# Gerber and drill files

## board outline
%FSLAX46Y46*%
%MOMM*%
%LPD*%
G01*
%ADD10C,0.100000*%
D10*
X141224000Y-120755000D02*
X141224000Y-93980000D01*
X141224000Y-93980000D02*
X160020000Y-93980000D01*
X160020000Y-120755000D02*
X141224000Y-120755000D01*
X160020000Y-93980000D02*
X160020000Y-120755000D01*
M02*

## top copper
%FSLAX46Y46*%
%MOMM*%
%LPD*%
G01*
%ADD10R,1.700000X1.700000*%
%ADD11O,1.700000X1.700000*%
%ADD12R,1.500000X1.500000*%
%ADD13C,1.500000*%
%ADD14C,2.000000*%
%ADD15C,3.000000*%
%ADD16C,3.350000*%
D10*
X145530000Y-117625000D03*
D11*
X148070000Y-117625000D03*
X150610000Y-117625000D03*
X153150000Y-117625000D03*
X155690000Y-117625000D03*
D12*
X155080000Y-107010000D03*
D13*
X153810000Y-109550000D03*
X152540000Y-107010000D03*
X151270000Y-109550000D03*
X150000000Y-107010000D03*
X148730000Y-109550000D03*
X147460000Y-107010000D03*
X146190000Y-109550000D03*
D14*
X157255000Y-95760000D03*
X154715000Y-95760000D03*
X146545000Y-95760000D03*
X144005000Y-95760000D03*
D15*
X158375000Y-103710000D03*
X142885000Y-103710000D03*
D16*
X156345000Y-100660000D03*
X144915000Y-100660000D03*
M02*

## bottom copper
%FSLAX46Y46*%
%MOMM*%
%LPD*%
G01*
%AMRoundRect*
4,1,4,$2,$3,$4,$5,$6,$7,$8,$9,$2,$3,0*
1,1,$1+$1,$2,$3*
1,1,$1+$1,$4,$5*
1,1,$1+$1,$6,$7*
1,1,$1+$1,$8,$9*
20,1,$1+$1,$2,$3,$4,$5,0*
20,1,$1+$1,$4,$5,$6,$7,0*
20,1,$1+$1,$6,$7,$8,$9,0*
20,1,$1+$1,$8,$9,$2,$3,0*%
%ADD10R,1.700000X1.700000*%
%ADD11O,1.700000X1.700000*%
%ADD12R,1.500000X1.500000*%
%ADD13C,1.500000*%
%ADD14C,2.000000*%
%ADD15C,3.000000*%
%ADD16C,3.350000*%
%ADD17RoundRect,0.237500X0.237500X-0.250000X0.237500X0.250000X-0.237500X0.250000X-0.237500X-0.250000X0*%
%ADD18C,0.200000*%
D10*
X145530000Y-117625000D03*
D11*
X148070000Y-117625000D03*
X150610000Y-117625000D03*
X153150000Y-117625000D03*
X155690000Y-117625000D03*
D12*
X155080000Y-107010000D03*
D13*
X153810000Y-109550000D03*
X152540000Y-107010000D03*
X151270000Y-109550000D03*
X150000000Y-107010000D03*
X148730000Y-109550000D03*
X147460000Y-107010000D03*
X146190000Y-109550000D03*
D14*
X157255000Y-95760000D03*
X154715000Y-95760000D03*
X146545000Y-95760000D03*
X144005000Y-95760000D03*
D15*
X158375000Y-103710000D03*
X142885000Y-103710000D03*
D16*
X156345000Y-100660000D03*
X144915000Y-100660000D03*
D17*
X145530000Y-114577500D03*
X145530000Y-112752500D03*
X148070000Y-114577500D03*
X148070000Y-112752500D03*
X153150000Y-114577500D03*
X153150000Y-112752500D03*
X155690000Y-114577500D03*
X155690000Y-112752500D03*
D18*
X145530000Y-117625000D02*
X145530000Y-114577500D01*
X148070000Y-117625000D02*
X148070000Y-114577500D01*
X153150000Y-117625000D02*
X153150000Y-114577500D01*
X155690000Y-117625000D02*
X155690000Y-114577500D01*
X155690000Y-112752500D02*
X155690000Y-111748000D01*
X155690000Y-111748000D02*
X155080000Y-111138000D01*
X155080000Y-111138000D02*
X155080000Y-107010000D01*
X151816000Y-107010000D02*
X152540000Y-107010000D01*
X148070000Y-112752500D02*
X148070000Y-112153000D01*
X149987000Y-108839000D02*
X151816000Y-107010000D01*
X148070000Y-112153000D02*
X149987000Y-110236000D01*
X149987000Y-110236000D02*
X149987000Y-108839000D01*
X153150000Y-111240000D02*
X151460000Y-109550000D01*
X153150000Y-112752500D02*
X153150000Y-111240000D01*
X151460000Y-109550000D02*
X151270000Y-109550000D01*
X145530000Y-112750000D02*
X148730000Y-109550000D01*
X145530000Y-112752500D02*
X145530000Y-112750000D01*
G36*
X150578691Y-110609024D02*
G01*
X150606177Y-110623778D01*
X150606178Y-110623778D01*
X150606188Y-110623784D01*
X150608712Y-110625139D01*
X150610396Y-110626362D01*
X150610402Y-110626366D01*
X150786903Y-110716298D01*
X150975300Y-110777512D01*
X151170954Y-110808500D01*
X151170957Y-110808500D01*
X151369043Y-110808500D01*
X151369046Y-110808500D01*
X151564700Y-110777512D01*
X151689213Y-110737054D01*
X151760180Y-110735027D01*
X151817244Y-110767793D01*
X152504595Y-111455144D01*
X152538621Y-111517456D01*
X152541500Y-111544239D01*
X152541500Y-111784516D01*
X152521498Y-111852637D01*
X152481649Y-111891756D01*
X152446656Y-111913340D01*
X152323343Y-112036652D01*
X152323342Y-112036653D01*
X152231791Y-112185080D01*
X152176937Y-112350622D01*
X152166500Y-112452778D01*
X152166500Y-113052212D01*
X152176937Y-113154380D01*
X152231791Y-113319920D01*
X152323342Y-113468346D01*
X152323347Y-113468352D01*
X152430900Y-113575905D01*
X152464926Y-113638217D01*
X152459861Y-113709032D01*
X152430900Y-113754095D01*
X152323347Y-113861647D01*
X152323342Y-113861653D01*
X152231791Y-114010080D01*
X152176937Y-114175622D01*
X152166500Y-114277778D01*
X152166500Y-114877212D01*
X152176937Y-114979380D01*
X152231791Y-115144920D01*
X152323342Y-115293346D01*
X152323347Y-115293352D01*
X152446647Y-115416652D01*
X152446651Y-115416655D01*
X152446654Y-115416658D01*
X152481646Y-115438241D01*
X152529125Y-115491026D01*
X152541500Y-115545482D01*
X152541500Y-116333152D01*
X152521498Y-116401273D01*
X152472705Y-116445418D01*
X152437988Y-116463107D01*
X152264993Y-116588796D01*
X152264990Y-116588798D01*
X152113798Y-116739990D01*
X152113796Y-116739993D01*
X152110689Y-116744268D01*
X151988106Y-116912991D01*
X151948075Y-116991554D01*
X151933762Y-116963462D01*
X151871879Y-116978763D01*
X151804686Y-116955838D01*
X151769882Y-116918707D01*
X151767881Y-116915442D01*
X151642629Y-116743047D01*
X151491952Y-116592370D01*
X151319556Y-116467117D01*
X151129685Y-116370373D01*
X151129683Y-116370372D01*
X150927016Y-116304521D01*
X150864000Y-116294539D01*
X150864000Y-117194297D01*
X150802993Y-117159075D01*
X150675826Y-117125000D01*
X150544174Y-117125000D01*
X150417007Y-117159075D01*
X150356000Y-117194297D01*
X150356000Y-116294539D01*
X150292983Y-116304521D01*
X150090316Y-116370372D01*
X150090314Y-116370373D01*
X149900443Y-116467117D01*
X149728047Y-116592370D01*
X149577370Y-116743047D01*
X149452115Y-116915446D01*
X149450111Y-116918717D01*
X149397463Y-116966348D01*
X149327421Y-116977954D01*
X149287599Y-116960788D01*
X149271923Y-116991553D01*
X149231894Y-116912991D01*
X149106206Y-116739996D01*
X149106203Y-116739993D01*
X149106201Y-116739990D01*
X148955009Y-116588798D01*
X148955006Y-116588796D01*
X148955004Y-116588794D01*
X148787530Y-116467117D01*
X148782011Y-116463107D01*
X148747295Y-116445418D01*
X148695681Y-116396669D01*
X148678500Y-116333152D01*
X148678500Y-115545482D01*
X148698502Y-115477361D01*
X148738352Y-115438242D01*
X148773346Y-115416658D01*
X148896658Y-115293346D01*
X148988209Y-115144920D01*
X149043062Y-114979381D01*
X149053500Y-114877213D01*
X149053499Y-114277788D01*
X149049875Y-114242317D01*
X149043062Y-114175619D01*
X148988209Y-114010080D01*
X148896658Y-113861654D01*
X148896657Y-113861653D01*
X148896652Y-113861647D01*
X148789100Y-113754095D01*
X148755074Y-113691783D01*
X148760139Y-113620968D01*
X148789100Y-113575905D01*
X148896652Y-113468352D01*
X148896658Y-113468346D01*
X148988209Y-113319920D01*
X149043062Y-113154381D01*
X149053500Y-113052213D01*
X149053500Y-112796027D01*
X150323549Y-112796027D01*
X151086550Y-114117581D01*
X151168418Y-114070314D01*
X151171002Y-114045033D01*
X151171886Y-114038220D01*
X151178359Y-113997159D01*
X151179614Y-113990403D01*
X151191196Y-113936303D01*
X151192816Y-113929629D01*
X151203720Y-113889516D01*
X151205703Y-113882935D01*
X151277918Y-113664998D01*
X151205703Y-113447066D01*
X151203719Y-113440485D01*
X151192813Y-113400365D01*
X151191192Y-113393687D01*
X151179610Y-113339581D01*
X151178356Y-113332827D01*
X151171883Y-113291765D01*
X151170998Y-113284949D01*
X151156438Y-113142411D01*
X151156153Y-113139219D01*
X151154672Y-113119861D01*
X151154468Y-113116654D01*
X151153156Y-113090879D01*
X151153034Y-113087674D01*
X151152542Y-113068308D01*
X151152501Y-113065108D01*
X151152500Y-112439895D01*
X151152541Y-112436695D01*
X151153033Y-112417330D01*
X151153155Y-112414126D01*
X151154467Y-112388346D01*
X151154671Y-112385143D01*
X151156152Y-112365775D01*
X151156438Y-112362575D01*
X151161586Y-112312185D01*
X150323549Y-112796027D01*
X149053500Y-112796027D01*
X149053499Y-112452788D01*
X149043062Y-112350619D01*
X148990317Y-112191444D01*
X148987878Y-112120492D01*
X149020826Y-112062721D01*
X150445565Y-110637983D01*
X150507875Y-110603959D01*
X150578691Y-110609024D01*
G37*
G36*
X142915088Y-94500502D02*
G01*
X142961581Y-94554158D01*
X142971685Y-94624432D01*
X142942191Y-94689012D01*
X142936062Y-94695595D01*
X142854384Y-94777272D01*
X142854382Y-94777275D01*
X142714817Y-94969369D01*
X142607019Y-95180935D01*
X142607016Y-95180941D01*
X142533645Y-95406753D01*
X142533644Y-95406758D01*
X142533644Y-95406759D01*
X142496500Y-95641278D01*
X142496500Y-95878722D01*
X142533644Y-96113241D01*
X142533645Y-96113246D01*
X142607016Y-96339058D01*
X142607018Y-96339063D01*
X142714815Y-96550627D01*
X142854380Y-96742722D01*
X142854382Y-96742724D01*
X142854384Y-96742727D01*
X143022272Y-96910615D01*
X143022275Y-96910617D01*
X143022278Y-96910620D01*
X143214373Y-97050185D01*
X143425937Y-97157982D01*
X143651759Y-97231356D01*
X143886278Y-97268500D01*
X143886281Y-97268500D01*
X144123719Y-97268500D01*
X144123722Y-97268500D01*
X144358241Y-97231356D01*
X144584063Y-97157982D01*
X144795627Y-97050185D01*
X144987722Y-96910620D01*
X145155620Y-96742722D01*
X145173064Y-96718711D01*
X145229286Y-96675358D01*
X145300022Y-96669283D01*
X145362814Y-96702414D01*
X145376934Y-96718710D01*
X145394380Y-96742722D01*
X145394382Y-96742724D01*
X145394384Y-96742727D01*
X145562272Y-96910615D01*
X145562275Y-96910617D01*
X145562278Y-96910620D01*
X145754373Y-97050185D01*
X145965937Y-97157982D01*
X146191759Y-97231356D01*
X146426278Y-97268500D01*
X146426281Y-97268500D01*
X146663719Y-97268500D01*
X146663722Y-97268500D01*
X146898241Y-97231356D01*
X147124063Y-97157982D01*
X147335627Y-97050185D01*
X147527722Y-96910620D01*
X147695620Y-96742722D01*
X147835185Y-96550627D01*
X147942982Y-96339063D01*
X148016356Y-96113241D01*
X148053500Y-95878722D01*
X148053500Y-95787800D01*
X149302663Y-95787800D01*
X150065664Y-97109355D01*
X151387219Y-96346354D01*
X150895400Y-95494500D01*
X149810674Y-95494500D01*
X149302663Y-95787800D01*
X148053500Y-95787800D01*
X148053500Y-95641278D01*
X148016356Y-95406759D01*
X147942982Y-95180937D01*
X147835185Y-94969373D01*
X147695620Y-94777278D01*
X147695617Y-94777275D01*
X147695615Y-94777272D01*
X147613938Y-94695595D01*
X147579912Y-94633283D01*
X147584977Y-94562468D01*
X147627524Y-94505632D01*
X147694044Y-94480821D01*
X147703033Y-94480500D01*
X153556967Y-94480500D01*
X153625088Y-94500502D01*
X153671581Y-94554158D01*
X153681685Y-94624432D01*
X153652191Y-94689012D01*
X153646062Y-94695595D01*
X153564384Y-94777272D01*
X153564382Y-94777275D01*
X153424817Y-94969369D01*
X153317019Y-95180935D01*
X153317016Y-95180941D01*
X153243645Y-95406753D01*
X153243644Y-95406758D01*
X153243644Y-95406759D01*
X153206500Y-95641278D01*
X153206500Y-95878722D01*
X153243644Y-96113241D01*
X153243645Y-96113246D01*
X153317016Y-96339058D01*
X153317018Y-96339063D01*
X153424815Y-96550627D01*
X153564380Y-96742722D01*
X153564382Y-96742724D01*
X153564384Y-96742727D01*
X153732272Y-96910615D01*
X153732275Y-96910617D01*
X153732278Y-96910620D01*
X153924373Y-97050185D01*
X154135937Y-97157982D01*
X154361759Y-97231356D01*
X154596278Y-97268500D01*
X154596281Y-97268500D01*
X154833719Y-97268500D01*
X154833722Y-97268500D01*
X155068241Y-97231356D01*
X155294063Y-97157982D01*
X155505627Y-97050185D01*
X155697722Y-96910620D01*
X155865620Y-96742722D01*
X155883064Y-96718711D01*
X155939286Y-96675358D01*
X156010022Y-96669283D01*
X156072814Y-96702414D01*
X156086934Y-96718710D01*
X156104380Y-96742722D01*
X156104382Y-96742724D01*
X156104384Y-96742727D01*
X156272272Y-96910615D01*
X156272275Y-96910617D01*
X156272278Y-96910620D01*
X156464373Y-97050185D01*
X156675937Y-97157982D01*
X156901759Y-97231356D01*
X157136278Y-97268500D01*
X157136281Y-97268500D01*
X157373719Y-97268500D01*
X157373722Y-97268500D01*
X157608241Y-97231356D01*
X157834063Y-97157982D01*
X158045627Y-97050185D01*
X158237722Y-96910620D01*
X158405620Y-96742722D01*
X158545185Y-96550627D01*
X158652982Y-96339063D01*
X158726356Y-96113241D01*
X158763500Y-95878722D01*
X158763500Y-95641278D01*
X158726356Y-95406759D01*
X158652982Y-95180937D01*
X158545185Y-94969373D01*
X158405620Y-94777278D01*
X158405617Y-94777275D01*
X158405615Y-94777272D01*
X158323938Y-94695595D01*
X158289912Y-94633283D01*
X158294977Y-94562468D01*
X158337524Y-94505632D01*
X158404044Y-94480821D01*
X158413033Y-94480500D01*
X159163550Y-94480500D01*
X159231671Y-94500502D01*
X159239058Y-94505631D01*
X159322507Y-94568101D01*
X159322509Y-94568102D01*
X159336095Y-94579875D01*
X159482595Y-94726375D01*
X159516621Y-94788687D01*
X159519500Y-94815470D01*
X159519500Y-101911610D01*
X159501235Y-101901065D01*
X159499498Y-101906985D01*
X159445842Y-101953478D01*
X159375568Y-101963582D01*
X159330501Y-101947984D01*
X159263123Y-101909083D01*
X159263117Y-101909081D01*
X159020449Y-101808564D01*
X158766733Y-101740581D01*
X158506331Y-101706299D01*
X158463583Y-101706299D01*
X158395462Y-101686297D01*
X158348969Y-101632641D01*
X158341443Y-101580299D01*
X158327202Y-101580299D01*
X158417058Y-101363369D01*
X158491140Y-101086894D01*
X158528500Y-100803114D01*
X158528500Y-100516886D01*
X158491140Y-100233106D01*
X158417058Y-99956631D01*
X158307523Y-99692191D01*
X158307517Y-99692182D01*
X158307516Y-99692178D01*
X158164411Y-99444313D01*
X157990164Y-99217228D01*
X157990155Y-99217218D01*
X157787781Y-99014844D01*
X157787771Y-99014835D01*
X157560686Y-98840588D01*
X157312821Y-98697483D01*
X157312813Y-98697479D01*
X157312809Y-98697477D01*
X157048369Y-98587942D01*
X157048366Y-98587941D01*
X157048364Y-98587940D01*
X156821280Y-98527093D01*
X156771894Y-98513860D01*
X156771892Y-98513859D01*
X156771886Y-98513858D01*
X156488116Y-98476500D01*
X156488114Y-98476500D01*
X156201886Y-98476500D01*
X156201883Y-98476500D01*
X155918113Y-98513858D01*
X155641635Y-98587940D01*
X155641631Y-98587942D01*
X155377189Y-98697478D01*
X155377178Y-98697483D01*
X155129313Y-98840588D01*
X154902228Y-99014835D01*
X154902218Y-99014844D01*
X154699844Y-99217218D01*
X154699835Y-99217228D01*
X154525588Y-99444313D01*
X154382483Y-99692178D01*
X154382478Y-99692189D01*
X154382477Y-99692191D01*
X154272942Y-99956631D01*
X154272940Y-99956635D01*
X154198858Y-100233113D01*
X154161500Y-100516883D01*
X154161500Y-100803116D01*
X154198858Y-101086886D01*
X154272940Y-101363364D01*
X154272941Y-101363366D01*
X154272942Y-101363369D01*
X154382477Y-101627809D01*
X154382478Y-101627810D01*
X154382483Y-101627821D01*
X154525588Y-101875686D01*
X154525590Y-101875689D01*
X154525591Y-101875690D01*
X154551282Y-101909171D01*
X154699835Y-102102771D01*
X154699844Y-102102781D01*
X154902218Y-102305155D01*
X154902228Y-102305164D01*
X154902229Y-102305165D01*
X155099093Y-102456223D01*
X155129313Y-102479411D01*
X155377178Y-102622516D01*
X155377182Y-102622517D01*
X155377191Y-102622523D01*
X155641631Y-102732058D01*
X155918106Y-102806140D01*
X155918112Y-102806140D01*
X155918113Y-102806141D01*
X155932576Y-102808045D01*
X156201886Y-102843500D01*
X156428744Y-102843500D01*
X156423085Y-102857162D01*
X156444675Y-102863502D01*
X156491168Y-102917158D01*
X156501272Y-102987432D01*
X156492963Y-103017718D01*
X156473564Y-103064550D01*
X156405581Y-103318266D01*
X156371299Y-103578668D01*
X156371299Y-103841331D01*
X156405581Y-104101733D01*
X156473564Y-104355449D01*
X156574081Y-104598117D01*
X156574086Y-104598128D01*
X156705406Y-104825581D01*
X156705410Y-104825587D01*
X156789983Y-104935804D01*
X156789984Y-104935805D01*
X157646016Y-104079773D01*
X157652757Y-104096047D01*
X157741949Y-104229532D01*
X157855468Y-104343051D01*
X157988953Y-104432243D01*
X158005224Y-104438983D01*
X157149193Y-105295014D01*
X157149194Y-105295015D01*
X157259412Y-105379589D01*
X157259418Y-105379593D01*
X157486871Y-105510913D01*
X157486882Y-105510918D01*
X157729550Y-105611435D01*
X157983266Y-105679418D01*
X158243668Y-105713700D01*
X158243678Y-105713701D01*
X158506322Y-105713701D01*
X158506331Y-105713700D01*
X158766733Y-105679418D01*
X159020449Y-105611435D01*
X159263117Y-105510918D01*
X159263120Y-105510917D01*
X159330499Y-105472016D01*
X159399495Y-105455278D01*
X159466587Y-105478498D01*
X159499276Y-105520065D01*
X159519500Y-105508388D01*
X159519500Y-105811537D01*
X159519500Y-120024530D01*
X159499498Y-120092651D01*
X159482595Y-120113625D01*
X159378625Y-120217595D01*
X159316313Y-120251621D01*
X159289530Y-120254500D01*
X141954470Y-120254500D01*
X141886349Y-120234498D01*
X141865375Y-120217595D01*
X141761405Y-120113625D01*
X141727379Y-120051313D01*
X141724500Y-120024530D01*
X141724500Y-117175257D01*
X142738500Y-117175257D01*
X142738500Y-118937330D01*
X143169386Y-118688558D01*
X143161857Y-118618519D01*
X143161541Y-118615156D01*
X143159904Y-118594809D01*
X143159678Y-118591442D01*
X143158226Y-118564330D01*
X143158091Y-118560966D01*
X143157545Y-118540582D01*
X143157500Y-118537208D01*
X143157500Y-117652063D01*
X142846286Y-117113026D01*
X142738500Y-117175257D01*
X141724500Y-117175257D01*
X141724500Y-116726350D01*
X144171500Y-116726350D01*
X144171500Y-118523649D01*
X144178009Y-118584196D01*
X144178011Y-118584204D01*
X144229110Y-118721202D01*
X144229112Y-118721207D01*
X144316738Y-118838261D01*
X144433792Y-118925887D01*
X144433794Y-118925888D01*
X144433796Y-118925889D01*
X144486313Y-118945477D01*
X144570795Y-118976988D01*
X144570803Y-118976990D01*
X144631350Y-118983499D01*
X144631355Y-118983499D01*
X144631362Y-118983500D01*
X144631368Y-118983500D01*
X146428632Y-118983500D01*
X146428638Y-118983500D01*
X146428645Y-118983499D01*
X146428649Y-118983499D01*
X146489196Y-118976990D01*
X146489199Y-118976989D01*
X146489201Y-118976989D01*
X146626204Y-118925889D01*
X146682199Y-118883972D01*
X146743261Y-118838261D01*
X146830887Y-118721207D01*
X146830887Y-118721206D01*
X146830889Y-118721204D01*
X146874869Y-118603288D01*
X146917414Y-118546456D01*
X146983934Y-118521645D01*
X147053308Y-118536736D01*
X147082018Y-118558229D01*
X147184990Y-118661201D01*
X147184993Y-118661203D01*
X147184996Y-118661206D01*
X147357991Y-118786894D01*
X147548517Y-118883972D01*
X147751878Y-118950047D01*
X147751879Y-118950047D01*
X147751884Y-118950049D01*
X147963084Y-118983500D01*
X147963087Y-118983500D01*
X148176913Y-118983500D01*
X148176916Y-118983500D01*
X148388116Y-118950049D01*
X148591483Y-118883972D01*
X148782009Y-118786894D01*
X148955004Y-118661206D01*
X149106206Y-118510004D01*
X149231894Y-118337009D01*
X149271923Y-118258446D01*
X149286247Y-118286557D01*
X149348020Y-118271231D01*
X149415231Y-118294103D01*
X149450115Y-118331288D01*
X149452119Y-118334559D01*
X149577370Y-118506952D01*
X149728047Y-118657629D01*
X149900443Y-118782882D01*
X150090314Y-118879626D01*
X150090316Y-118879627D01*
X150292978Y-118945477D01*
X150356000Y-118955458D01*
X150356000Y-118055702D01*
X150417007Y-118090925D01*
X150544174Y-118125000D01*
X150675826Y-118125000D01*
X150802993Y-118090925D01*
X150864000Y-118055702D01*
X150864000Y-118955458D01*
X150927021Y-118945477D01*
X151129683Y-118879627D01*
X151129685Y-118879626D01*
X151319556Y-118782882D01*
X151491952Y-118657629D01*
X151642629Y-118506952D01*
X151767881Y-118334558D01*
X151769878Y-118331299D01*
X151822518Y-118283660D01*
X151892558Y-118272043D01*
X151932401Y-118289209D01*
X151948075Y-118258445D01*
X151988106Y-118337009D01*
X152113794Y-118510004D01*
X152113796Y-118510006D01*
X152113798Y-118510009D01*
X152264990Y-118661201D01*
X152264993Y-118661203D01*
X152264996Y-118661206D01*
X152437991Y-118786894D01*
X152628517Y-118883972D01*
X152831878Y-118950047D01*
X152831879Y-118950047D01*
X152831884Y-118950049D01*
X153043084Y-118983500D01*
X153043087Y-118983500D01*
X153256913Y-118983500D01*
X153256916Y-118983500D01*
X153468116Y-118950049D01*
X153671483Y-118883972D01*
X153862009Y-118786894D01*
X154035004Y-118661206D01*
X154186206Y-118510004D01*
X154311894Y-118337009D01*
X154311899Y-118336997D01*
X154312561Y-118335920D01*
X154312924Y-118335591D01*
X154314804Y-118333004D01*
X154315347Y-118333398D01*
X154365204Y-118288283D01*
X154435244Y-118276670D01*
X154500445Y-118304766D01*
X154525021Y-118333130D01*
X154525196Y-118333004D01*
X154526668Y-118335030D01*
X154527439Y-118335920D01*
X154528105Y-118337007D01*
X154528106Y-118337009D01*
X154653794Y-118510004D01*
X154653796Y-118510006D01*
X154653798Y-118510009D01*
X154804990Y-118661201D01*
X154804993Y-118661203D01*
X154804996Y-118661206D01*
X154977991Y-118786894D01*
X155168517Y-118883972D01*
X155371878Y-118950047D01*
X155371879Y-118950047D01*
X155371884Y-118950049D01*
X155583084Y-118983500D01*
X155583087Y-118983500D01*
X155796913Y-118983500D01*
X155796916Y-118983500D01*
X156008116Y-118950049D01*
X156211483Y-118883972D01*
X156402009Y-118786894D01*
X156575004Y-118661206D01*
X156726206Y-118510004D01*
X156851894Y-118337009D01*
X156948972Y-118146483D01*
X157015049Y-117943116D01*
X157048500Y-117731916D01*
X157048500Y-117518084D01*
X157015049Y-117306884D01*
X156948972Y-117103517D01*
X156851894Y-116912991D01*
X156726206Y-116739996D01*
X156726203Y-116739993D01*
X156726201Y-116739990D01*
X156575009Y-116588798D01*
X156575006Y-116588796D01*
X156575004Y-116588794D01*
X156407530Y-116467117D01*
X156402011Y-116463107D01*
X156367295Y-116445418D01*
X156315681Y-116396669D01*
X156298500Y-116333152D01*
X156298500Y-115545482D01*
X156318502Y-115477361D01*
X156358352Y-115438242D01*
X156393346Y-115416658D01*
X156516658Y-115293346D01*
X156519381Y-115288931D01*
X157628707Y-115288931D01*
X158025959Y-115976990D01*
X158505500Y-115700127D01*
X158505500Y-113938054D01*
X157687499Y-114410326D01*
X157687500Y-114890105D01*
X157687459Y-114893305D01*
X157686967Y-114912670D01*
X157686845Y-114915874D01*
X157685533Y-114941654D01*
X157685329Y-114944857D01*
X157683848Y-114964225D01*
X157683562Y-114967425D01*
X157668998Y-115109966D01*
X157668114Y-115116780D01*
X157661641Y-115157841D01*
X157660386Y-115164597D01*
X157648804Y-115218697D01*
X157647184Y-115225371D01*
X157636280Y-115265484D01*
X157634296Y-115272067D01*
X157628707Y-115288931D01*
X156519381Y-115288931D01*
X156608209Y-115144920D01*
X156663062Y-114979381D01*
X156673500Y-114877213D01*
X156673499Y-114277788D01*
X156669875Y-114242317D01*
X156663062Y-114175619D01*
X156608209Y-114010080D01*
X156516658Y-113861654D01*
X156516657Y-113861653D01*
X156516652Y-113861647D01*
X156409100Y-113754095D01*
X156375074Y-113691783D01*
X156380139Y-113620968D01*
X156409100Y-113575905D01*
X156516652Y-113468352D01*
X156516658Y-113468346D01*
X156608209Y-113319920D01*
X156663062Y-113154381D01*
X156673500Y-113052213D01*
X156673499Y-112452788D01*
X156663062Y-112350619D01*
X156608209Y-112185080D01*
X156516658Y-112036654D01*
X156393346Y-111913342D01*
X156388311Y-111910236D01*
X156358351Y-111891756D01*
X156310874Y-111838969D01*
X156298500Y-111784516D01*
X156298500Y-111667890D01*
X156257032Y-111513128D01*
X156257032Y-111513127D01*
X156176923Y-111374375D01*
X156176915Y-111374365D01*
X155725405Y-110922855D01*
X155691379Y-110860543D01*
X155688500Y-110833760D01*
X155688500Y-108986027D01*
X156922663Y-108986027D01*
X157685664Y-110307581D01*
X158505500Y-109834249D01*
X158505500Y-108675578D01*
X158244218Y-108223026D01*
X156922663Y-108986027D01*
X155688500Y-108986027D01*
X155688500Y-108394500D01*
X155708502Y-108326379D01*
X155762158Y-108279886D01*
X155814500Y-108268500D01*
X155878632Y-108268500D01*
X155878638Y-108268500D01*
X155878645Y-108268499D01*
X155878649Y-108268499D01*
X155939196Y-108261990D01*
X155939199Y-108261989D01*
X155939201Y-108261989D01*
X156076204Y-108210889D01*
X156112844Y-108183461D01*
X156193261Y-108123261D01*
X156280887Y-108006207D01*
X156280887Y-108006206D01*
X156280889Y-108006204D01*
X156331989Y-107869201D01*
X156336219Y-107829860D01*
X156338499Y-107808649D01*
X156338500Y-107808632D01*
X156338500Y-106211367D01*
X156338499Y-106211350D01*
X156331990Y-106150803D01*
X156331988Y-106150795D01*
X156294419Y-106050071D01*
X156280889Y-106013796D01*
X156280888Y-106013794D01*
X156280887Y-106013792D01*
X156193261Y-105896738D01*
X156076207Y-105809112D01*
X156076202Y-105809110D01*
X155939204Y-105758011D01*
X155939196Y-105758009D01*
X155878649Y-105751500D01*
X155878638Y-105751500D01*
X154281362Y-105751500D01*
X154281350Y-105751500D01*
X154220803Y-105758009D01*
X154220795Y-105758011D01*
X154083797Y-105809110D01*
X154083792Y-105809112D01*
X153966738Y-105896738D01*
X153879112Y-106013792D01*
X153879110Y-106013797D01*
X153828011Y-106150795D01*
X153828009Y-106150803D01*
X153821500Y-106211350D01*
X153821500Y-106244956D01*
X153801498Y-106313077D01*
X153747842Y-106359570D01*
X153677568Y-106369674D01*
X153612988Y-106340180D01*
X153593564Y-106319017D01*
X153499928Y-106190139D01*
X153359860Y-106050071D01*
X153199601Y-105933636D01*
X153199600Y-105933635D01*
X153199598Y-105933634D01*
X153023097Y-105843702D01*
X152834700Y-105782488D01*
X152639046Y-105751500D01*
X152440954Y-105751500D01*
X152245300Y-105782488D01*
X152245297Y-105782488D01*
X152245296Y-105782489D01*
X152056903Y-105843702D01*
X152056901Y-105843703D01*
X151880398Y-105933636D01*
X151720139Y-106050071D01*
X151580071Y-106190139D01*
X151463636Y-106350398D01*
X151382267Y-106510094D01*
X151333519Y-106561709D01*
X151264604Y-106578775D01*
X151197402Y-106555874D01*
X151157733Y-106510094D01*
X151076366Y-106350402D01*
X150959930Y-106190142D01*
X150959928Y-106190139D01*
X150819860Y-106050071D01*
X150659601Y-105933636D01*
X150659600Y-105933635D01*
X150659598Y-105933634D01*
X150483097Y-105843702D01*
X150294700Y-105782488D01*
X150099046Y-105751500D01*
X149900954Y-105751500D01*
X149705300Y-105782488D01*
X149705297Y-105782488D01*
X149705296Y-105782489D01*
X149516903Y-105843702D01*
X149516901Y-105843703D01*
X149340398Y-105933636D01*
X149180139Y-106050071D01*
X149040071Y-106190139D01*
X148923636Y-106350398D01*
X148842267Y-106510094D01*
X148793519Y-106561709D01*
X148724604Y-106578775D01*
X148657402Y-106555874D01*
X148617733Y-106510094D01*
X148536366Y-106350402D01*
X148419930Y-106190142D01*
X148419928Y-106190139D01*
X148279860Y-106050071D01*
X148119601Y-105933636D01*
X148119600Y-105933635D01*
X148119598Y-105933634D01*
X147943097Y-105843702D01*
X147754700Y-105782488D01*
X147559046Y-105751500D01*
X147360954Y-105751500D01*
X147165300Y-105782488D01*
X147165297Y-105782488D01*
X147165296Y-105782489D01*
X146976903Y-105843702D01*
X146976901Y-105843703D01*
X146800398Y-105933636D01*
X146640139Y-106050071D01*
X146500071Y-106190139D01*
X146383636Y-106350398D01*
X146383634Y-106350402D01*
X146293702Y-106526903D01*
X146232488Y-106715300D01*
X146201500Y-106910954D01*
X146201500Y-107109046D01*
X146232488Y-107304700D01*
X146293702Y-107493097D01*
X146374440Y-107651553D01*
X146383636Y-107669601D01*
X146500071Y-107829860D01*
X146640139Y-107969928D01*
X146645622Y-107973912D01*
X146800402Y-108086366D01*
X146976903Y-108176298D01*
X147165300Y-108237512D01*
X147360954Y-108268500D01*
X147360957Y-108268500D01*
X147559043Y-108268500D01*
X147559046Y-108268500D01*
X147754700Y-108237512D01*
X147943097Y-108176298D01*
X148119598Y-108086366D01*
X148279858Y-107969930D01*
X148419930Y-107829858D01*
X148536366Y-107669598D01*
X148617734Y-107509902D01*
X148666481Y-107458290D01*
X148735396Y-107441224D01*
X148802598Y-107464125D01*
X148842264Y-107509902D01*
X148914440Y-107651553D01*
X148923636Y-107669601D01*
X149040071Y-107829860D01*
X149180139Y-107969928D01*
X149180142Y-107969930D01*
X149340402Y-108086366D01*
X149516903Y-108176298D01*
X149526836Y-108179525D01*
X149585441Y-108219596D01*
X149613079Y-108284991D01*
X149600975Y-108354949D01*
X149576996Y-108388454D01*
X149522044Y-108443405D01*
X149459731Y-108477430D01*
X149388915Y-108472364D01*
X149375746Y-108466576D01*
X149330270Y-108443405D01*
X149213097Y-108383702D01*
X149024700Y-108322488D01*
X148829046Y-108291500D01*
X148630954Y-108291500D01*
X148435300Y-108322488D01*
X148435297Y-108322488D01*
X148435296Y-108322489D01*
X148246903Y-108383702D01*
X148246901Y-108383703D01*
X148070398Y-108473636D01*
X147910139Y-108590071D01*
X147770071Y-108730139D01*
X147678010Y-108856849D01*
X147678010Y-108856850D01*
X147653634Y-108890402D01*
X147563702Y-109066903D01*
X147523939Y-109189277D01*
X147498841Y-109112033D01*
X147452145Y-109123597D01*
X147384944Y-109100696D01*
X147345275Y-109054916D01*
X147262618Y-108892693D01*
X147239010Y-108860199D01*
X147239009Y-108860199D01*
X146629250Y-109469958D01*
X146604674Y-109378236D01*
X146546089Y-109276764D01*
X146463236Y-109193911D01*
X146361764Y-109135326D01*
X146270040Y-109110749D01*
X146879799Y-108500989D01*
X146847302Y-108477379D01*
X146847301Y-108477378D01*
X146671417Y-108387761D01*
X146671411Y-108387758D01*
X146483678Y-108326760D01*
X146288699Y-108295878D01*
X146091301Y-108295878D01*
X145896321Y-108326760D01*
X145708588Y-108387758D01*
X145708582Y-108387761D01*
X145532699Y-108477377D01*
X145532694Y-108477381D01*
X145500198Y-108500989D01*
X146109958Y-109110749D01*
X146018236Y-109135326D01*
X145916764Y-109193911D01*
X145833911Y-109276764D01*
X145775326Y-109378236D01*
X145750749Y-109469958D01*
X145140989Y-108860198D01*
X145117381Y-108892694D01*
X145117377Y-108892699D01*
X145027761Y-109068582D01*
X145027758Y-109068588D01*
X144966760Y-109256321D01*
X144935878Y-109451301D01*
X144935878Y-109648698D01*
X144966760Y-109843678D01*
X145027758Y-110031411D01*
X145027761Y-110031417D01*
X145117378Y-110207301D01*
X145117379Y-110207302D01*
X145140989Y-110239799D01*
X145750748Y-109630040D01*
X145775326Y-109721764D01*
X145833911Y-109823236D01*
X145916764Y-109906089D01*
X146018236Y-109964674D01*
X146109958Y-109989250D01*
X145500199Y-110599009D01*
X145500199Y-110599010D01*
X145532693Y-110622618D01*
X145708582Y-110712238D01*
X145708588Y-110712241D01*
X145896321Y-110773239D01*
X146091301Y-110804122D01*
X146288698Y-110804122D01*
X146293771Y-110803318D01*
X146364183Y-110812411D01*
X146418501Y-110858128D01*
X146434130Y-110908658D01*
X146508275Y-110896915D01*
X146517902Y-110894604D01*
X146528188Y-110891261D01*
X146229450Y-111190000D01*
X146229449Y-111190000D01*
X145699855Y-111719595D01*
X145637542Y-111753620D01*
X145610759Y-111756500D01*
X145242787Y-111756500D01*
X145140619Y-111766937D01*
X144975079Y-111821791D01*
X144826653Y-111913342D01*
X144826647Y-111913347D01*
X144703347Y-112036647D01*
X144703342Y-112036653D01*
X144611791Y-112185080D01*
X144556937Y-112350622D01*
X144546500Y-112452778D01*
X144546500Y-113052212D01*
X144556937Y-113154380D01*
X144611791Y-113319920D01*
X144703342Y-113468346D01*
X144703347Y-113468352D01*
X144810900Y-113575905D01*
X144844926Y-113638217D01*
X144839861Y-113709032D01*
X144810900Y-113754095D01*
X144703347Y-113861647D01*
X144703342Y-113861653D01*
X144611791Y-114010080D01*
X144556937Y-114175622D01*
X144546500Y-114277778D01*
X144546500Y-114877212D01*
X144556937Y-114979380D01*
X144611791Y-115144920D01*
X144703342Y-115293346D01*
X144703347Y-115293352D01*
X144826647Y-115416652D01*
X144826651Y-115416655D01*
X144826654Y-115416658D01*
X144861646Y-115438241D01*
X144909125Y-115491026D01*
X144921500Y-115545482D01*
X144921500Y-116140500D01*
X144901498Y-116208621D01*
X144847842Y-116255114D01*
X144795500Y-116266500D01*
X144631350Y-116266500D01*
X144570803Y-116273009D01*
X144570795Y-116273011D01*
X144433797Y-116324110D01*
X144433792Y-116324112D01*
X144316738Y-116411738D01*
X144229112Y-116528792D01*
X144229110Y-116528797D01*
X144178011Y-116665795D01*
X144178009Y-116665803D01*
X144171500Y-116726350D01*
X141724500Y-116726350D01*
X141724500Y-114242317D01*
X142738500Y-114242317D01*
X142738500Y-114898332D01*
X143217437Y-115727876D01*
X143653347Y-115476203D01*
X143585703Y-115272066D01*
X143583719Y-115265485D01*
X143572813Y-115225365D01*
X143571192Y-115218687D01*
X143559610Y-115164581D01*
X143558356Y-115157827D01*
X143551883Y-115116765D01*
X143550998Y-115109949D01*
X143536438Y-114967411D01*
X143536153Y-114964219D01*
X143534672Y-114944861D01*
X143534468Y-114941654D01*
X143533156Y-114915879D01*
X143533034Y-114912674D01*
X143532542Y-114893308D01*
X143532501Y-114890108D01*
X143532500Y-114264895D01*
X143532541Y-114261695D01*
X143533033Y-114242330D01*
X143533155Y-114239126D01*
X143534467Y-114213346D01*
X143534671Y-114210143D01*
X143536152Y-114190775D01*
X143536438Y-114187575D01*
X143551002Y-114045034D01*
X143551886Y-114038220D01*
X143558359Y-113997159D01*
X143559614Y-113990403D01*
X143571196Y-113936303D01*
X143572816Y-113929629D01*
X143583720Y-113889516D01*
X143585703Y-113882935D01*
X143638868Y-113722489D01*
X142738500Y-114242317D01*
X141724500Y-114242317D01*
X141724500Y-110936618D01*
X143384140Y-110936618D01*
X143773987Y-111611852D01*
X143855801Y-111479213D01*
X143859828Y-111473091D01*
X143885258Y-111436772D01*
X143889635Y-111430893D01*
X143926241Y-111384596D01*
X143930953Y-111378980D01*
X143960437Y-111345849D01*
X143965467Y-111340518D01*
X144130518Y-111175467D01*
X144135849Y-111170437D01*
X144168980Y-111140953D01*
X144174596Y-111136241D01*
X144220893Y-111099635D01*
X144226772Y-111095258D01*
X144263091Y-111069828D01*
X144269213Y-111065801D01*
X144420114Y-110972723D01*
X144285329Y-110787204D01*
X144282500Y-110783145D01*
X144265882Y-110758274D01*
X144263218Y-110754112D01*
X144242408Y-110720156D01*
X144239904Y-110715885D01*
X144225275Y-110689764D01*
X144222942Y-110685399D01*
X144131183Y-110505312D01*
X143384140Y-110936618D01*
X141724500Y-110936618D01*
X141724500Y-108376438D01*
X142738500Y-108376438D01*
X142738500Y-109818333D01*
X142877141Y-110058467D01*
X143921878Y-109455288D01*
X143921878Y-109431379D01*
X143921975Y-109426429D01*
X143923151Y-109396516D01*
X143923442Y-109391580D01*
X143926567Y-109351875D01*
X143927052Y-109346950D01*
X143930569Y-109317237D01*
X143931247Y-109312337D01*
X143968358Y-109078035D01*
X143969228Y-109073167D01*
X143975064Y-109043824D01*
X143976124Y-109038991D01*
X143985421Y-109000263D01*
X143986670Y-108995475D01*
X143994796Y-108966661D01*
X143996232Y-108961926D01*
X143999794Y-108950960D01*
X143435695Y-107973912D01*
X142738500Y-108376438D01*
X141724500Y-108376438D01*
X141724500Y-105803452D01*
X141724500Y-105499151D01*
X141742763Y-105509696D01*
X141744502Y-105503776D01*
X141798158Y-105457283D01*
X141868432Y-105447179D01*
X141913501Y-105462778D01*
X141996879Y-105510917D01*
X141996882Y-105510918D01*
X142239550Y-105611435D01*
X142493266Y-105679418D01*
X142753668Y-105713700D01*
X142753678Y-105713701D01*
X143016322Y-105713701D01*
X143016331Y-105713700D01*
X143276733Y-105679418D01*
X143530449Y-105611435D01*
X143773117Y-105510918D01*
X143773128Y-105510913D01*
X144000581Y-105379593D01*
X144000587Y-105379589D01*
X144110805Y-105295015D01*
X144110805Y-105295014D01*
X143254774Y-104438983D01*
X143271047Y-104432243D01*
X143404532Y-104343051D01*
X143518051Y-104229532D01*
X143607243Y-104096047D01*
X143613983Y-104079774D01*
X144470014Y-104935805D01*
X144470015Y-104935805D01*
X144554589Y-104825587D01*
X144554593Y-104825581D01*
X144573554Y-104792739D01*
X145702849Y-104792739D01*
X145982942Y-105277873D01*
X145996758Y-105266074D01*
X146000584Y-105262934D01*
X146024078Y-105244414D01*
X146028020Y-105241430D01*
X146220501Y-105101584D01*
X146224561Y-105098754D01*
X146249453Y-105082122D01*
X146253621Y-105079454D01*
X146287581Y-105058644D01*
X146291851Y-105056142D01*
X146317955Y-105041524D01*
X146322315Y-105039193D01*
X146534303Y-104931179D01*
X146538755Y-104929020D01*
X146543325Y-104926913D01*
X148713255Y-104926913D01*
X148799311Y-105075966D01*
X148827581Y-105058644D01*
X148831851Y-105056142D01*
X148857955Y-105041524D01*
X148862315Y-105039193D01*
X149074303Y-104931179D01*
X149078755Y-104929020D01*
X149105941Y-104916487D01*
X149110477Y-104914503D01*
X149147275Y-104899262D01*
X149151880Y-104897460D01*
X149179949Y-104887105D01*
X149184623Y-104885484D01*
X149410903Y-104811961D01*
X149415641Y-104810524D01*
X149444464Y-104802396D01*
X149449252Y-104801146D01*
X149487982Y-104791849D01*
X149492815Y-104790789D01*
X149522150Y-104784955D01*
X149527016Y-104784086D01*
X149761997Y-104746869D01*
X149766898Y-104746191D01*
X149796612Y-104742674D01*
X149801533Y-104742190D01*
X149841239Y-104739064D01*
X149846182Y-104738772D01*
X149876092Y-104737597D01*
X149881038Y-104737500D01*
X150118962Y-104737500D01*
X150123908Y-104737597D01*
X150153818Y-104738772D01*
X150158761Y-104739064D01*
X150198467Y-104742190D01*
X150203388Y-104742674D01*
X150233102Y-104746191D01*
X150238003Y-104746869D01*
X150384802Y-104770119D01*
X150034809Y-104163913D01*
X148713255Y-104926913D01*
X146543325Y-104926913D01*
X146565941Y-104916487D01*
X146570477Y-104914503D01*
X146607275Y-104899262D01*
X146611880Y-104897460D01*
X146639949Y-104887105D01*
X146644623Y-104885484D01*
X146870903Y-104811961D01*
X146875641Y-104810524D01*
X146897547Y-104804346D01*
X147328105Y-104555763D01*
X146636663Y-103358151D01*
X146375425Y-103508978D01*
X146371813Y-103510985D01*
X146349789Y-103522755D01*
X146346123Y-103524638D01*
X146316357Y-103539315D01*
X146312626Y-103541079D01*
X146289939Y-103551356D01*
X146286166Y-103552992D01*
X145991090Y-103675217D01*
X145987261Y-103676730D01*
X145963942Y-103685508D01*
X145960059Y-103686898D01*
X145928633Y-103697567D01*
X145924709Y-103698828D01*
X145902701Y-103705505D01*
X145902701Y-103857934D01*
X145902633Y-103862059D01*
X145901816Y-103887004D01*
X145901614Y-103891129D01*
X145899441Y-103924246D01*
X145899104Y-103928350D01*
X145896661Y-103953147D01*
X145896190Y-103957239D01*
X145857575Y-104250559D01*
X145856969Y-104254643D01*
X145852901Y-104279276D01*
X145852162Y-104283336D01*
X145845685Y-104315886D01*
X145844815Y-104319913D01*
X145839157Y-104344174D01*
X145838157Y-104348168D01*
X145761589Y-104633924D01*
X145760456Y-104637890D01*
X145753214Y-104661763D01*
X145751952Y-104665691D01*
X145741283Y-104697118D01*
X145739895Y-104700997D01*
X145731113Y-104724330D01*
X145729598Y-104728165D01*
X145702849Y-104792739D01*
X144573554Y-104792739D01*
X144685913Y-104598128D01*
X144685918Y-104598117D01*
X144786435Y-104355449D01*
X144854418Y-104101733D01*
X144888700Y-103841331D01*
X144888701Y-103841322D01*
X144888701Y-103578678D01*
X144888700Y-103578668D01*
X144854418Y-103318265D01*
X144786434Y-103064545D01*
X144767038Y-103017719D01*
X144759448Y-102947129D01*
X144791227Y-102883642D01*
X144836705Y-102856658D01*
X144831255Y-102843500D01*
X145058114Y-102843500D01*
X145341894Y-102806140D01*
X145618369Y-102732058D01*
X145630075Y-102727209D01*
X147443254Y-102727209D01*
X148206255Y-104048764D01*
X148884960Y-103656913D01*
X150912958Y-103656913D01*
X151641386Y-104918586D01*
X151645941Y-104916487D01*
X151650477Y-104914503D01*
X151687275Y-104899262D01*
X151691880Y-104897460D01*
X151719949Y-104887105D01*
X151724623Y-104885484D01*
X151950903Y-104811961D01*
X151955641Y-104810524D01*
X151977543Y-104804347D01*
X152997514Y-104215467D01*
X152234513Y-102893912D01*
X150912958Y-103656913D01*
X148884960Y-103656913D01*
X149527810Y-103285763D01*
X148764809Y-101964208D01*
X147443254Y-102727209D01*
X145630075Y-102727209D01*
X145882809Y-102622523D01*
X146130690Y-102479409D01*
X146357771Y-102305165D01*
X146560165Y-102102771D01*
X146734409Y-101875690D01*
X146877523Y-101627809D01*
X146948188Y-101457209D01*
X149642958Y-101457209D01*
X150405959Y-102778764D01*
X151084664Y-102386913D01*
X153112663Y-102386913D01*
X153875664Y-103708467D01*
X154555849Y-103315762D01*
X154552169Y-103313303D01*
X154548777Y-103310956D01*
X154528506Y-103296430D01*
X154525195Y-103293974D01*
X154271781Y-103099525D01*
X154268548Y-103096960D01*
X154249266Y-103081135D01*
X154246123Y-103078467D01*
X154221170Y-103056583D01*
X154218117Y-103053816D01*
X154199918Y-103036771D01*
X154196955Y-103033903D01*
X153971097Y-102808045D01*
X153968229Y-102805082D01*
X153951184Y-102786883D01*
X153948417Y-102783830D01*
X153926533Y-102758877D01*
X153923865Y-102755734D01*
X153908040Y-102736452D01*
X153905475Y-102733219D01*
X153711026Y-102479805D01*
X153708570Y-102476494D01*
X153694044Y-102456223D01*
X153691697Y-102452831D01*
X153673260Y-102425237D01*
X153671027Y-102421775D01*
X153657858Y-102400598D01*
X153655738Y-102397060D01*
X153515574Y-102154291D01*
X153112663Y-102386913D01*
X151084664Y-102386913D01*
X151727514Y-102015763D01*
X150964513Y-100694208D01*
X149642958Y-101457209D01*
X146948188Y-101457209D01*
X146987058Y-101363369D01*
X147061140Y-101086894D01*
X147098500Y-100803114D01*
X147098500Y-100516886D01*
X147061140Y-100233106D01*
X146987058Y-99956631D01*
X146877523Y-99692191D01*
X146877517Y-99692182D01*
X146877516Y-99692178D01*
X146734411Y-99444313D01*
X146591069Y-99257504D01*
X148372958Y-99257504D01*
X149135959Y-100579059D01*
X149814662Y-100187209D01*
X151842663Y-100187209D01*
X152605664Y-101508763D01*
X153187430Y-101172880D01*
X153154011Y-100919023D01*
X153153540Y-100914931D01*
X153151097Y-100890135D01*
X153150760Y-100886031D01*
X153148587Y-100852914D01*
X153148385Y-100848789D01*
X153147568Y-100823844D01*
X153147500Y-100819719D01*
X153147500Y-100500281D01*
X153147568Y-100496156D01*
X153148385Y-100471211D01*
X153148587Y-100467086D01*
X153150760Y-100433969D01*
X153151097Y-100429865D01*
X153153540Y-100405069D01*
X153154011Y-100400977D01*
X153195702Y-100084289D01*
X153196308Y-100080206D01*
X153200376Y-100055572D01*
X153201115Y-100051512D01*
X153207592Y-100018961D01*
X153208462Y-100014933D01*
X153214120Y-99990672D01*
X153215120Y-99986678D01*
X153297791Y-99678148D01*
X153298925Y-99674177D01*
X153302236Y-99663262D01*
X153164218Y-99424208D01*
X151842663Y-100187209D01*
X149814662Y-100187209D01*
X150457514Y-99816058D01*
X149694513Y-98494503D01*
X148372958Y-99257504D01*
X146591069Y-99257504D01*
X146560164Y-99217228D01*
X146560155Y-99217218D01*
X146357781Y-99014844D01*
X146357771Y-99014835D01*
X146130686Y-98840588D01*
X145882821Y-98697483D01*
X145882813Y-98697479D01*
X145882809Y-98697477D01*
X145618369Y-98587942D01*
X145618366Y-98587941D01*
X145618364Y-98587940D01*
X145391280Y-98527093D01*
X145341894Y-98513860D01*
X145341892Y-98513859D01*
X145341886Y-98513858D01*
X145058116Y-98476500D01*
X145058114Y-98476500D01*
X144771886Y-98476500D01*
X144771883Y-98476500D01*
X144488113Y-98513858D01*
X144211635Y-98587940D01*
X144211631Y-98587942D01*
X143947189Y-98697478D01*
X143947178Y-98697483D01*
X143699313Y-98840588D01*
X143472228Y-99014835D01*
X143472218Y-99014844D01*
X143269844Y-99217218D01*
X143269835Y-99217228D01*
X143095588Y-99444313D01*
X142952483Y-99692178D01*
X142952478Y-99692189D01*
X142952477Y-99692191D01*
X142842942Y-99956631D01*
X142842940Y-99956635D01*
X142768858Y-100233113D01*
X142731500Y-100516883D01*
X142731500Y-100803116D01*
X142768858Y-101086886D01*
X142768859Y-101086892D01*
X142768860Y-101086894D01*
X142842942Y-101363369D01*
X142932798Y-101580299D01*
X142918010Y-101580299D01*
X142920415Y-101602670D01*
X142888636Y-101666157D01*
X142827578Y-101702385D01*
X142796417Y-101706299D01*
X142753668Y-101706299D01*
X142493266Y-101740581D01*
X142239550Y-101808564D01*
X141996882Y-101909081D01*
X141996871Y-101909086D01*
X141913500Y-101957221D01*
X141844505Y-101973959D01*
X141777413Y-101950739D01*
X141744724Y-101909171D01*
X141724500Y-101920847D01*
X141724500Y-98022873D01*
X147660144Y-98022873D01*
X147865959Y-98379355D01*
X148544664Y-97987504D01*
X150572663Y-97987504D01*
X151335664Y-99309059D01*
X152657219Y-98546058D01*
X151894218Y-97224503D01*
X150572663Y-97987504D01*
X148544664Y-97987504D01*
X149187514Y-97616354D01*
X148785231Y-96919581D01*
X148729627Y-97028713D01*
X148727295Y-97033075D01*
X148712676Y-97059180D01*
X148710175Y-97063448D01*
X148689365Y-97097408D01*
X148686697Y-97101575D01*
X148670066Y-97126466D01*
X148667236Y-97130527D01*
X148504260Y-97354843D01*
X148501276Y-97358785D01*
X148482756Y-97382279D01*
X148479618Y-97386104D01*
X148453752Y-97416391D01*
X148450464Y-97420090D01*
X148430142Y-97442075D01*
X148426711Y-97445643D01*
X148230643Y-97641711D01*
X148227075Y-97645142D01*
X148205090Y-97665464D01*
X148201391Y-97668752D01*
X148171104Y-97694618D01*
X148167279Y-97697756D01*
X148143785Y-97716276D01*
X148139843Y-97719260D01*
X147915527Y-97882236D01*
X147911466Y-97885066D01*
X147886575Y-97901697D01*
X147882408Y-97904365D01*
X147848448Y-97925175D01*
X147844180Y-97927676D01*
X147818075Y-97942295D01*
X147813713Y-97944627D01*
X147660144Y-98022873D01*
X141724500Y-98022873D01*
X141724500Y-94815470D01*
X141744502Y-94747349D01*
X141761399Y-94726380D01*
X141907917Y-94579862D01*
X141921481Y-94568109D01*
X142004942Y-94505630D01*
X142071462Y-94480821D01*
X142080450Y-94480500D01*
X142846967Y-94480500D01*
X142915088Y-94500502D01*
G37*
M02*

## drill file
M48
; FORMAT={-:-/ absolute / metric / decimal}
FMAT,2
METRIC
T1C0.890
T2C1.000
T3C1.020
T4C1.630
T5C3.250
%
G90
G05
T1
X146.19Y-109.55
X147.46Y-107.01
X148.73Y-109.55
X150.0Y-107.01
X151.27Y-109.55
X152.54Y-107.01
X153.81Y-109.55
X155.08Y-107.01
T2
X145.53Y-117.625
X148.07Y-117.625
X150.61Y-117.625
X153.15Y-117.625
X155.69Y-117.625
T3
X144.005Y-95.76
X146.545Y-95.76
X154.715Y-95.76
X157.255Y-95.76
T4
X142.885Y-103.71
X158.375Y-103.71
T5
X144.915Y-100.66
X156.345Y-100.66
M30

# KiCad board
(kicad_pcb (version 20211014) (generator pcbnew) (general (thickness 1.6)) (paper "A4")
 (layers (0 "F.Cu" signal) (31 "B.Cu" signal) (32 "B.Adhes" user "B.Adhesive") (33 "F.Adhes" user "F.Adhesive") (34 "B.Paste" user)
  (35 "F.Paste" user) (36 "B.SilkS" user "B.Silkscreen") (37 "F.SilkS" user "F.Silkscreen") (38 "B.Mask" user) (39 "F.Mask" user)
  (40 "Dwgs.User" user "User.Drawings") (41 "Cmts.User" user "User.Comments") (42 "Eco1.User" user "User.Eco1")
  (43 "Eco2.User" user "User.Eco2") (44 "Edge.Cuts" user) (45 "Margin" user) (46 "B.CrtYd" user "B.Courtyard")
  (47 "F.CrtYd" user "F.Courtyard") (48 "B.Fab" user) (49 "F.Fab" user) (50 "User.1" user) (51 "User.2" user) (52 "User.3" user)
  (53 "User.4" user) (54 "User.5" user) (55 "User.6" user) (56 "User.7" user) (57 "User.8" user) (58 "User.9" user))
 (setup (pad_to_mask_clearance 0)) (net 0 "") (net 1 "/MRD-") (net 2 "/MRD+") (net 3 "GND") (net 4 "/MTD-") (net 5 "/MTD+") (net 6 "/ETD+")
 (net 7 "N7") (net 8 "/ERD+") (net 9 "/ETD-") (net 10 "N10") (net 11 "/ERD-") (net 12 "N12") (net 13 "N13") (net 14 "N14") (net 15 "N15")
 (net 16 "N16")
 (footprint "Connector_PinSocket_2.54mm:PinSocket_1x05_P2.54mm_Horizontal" (layer "F.Cu") (at 145.53 117.625 90)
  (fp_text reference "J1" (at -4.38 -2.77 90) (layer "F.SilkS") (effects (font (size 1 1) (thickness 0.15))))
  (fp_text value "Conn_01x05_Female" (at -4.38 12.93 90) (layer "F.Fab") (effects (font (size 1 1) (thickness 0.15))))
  (pad "1" thru_hole rect (at 0 0 90) (size 1.7 1.7) (drill 1) (layers *.Cu *.Mask) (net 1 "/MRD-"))
  (pad "2" thru_hole oval (at 0 2.54 90) (size 1.7 1.7) (drill 1) (layers *.Cu *.Mask) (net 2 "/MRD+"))
  (pad "3" thru_hole oval (at 0 5.08 90) (size 1.7 1.7) (drill 1) (layers *.Cu *.Mask) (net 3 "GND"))
  (pad "4" thru_hole oval (at 0 7.62 90) (size 1.7 1.7) (drill 1) (layers *.Cu *.Mask) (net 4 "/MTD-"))
  (pad "5" thru_hole oval (at 0 10.16 90) (size 1.7 1.7) (drill 1) (layers *.Cu *.Mask) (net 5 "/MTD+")))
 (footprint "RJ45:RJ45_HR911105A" (layer "F.Cu") (at 150.63 100.66)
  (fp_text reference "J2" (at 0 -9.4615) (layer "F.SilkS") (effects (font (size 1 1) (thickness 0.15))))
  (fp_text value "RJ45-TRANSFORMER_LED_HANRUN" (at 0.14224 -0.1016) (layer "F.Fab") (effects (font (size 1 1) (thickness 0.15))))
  (pad "1" thru_hole rect (at 4.45 6.35) (size 1.5 1.5) (drill 0.89) (layers *.Cu *.Mask "F.SilkS") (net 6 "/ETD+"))
  (pad "2" thru_hole circle (at 3.18 8.89) (size 1.5 1.5) (drill 0.89) (layers *.Cu *.Mask "F.SilkS") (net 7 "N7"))
  (pad "3" thru_hole circle (at 1.91 6.35) (size 1.5 1.5) (drill 0.89) (layers *.Cu *.Mask "F.SilkS") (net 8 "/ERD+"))
  (pad "4" thru_hole circle (at 0.64 8.89) (size 1.5 1.5) (drill 0.89) (layers *.Cu *.Mask "F.SilkS") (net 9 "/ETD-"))
  (pad "5" thru_hole circle (at -0.63 6.35) (size 1.5 1.5) (drill 0.89) (layers *.Cu *.Mask "F.SilkS") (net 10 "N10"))
  (pad "6" thru_hole circle (at -1.9 8.89) (size 1.5 1.5) (drill 0.89) (layers *.Cu *.Mask "F.SilkS") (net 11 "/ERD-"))
  (pad "7" thru_hole circle (at -3.17 6.35) (size 1.5 1.5) (drill 0.89) (layers *.Cu *.Mask "F.SilkS") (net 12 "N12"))
  (pad "8" thru_hole circle (at -4.44 8.89) (size 1.5 1.5) (drill 0.89) (layers *.Cu *.Mask "F.SilkS") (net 3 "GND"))
  (pad "9" thru_hole circle (at 6.625 -4.9) (size 2 2) (drill 1.02) (layers *.Cu *.SilkS *.Mask) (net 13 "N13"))
  (pad "10" thru_hole circle (at 4.085 -4.9) (size 2 2) (drill 1.02) (layers *.Cu *.SilkS *.Mask) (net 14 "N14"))
  (pad "11" thru_hole circle (at -4.085 -4.9) (size 2 2) (drill 1.02) (layers *.Cu *.SilkS *.Mask) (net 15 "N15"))
  (pad "12" thru_hole circle (at -6.625 -4.9) (size 2 2) (drill 1.02) (layers *.Cu *.SilkS *.Mask) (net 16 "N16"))
  (pad "13" thru_hole circle (at 7.745 3.05) (size 3 3) (drill 1.63) (layers *.Cu *.SilkS *.Mask) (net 3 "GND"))
  (pad "13" thru_hole circle (at -7.745 3.05) (size 3 3) (drill 1.63) (layers *.Cu *.SilkS *.Mask) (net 3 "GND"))
  (pad "Hole" thru_hole circle (at 5.715 0) (size 3.35 3.35) (drill 3.25) (layers *.Cu *.SilkS *.Mask))
  (pad "Hole" thru_hole circle (at -5.715 0) (size 3.35 3.35) (drill 3.25) (layers *.Cu *.SilkS *.Mask)))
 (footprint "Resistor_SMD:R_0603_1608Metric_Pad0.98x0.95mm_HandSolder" (layer "B.Cu") (at 145.53 113.665 90)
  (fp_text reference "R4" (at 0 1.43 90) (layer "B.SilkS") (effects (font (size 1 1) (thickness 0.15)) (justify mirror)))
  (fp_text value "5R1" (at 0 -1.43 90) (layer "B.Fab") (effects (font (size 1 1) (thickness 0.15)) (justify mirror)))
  (pad "1" smd roundrect (at -0.9125 0 90) (size 0.975 0.95) (layers "B.Cu" "B.Paste" "B.Mask") (roundrect_rratio 0.25) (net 1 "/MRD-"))
  (pad "2" smd roundrect (at 0.9125 0 90) (size 0.975 0.95) (layers "B.Cu" "B.Paste" "B.Mask") (roundrect_rratio 0.25) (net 11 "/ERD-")))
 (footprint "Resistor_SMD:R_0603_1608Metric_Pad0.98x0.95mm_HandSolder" (layer "B.Cu") (at 148.07 113.665 90)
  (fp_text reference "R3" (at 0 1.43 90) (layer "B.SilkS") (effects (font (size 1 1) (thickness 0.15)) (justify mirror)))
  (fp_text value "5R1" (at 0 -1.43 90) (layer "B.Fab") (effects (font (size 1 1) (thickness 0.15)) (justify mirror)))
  (pad "1" smd roundrect (at -0.9125 0 90) (size 0.975 0.95) (layers "B.Cu" "B.Paste" "B.Mask") (roundrect_rratio 0.25) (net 2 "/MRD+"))
  (pad "2" smd roundrect (at 0.9125 0 90) (size 0.975 0.95) (layers "B.Cu" "B.Paste" "B.Mask") (roundrect_rratio 0.25) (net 8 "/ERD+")))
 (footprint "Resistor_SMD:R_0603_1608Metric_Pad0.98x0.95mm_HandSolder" (layer "B.Cu") (at 153.15 113.665 90)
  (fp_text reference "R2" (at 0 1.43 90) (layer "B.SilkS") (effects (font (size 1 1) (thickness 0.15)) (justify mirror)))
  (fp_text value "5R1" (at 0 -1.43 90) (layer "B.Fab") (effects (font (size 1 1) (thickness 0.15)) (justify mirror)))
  (pad "1" smd roundrect (at -0.9125 0 90) (size 0.975 0.95) (layers "B.Cu" "B.Paste" "B.Mask") (roundrect_rratio 0.25) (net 4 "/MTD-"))
  (pad "2" smd roundrect (at 0.9125 0 90) (size 0.975 0.95) (layers "B.Cu" "B.Paste" "B.Mask") (roundrect_rratio 0.25) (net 9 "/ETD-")))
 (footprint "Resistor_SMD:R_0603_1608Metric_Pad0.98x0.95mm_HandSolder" (layer "B.Cu") (at 155.69 113.665 90)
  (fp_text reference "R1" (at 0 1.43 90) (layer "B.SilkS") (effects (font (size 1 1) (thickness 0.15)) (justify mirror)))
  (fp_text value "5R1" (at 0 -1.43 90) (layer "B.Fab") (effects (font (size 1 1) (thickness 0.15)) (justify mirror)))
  (pad "1" smd roundrect (at -0.9125 0 90) (size 0.975 0.95) (layers "B.Cu" "B.Paste" "B.Mask") (roundrect_rratio 0.25) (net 5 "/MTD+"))
  (pad "2" smd roundrect (at 0.9125 0 90) (size 0.975 0.95) (layers "B.Cu" "B.Paste" "B.Mask") (roundrect_rratio 0.25) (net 6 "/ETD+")))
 (gr_line (start 141.224 120.755) (end 141.224 93.98) (layer "Edge.Cuts") (width 0.1))
 (gr_line (start 141.224 93.98) (end 160.02 93.98) (layer "Edge.Cuts") (width 0.1))
 (gr_line (start 160.02 120.755) (end 141.224 120.755) (layer "Edge.Cuts") (width 0.1))
 (gr_line (start 160.02 93.98) (end 160.02 120.755) (layer "Edge.Cuts") (width 0.1))
 (segment (start 145.53 117.625) (end 145.53 114.5775) (width 0.2) (layer "B.Cu") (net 1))
 (segment (start 148.07 117.625) (end 148.07 114.5775) (width 0.2) (layer "B.Cu") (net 2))
 (segment (start 153.15 117.625) (end 153.15 114.5775) (width 0.2) (layer "B.Cu") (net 4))
 (segment (start 155.69 117.625) (end 155.69 114.5775) (width 0.2) (layer "B.Cu") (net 5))
 (segment (start 155.69 112.7525) (end 155.69 111.748) (width 0.2) (layer "B.Cu") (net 6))
 (segment (start 155.69 111.748) (end 155.08 111.138) (width 0.2) (layer "B.Cu") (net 6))
 (segment (start 155.08 111.138) (end 155.08 107.01) (width 0.2) (layer "B.Cu") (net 6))
 (segment (start 151.816 107.01) (end 152.54 107.01) (width 0.2) (layer "B.Cu") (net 8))
 (segment (start 148.07 112.7525) (end 148.07 112.153) (width 0.2) (layer "B.Cu") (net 8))
 (segment (start 149.987 108.839) (end 151.816 107.01) (width 0.2) (layer "B.Cu") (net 8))
 (segment (start 148.07 112.153) (end 149.987 110.236) (width 0.2) (layer "B.Cu") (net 8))
 (segment (start 149.987 110.236) (end 149.987 108.839) (width 0.2) (layer "B.Cu") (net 8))
 (segment (start 153.15 111.24) (end 151.46 109.55) (width 0.2) (layer "B.Cu") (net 9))
 (segment (start 153.15 112.7525) (end 153.15 111.24) (width 0.2) (layer "B.Cu") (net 9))
 (segment (start 151.46 109.55) (end 151.27 109.55) (width 0.2) (layer "B.Cu") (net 9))
 (segment (start 145.53 112.75) (end 148.73 109.55) (width 0.2) (layer "B.Cu") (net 11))
 (segment (start 145.53 112.7525) (end 145.53 112.75) (width 0.2) (layer "B.Cu") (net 11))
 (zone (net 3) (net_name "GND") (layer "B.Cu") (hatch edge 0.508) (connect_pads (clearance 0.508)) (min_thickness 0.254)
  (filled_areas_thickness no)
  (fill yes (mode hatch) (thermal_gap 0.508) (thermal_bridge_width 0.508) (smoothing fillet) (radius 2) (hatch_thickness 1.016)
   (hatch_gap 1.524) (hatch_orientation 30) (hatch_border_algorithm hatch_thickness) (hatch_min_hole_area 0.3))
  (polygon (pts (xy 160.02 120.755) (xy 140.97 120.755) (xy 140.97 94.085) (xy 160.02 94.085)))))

